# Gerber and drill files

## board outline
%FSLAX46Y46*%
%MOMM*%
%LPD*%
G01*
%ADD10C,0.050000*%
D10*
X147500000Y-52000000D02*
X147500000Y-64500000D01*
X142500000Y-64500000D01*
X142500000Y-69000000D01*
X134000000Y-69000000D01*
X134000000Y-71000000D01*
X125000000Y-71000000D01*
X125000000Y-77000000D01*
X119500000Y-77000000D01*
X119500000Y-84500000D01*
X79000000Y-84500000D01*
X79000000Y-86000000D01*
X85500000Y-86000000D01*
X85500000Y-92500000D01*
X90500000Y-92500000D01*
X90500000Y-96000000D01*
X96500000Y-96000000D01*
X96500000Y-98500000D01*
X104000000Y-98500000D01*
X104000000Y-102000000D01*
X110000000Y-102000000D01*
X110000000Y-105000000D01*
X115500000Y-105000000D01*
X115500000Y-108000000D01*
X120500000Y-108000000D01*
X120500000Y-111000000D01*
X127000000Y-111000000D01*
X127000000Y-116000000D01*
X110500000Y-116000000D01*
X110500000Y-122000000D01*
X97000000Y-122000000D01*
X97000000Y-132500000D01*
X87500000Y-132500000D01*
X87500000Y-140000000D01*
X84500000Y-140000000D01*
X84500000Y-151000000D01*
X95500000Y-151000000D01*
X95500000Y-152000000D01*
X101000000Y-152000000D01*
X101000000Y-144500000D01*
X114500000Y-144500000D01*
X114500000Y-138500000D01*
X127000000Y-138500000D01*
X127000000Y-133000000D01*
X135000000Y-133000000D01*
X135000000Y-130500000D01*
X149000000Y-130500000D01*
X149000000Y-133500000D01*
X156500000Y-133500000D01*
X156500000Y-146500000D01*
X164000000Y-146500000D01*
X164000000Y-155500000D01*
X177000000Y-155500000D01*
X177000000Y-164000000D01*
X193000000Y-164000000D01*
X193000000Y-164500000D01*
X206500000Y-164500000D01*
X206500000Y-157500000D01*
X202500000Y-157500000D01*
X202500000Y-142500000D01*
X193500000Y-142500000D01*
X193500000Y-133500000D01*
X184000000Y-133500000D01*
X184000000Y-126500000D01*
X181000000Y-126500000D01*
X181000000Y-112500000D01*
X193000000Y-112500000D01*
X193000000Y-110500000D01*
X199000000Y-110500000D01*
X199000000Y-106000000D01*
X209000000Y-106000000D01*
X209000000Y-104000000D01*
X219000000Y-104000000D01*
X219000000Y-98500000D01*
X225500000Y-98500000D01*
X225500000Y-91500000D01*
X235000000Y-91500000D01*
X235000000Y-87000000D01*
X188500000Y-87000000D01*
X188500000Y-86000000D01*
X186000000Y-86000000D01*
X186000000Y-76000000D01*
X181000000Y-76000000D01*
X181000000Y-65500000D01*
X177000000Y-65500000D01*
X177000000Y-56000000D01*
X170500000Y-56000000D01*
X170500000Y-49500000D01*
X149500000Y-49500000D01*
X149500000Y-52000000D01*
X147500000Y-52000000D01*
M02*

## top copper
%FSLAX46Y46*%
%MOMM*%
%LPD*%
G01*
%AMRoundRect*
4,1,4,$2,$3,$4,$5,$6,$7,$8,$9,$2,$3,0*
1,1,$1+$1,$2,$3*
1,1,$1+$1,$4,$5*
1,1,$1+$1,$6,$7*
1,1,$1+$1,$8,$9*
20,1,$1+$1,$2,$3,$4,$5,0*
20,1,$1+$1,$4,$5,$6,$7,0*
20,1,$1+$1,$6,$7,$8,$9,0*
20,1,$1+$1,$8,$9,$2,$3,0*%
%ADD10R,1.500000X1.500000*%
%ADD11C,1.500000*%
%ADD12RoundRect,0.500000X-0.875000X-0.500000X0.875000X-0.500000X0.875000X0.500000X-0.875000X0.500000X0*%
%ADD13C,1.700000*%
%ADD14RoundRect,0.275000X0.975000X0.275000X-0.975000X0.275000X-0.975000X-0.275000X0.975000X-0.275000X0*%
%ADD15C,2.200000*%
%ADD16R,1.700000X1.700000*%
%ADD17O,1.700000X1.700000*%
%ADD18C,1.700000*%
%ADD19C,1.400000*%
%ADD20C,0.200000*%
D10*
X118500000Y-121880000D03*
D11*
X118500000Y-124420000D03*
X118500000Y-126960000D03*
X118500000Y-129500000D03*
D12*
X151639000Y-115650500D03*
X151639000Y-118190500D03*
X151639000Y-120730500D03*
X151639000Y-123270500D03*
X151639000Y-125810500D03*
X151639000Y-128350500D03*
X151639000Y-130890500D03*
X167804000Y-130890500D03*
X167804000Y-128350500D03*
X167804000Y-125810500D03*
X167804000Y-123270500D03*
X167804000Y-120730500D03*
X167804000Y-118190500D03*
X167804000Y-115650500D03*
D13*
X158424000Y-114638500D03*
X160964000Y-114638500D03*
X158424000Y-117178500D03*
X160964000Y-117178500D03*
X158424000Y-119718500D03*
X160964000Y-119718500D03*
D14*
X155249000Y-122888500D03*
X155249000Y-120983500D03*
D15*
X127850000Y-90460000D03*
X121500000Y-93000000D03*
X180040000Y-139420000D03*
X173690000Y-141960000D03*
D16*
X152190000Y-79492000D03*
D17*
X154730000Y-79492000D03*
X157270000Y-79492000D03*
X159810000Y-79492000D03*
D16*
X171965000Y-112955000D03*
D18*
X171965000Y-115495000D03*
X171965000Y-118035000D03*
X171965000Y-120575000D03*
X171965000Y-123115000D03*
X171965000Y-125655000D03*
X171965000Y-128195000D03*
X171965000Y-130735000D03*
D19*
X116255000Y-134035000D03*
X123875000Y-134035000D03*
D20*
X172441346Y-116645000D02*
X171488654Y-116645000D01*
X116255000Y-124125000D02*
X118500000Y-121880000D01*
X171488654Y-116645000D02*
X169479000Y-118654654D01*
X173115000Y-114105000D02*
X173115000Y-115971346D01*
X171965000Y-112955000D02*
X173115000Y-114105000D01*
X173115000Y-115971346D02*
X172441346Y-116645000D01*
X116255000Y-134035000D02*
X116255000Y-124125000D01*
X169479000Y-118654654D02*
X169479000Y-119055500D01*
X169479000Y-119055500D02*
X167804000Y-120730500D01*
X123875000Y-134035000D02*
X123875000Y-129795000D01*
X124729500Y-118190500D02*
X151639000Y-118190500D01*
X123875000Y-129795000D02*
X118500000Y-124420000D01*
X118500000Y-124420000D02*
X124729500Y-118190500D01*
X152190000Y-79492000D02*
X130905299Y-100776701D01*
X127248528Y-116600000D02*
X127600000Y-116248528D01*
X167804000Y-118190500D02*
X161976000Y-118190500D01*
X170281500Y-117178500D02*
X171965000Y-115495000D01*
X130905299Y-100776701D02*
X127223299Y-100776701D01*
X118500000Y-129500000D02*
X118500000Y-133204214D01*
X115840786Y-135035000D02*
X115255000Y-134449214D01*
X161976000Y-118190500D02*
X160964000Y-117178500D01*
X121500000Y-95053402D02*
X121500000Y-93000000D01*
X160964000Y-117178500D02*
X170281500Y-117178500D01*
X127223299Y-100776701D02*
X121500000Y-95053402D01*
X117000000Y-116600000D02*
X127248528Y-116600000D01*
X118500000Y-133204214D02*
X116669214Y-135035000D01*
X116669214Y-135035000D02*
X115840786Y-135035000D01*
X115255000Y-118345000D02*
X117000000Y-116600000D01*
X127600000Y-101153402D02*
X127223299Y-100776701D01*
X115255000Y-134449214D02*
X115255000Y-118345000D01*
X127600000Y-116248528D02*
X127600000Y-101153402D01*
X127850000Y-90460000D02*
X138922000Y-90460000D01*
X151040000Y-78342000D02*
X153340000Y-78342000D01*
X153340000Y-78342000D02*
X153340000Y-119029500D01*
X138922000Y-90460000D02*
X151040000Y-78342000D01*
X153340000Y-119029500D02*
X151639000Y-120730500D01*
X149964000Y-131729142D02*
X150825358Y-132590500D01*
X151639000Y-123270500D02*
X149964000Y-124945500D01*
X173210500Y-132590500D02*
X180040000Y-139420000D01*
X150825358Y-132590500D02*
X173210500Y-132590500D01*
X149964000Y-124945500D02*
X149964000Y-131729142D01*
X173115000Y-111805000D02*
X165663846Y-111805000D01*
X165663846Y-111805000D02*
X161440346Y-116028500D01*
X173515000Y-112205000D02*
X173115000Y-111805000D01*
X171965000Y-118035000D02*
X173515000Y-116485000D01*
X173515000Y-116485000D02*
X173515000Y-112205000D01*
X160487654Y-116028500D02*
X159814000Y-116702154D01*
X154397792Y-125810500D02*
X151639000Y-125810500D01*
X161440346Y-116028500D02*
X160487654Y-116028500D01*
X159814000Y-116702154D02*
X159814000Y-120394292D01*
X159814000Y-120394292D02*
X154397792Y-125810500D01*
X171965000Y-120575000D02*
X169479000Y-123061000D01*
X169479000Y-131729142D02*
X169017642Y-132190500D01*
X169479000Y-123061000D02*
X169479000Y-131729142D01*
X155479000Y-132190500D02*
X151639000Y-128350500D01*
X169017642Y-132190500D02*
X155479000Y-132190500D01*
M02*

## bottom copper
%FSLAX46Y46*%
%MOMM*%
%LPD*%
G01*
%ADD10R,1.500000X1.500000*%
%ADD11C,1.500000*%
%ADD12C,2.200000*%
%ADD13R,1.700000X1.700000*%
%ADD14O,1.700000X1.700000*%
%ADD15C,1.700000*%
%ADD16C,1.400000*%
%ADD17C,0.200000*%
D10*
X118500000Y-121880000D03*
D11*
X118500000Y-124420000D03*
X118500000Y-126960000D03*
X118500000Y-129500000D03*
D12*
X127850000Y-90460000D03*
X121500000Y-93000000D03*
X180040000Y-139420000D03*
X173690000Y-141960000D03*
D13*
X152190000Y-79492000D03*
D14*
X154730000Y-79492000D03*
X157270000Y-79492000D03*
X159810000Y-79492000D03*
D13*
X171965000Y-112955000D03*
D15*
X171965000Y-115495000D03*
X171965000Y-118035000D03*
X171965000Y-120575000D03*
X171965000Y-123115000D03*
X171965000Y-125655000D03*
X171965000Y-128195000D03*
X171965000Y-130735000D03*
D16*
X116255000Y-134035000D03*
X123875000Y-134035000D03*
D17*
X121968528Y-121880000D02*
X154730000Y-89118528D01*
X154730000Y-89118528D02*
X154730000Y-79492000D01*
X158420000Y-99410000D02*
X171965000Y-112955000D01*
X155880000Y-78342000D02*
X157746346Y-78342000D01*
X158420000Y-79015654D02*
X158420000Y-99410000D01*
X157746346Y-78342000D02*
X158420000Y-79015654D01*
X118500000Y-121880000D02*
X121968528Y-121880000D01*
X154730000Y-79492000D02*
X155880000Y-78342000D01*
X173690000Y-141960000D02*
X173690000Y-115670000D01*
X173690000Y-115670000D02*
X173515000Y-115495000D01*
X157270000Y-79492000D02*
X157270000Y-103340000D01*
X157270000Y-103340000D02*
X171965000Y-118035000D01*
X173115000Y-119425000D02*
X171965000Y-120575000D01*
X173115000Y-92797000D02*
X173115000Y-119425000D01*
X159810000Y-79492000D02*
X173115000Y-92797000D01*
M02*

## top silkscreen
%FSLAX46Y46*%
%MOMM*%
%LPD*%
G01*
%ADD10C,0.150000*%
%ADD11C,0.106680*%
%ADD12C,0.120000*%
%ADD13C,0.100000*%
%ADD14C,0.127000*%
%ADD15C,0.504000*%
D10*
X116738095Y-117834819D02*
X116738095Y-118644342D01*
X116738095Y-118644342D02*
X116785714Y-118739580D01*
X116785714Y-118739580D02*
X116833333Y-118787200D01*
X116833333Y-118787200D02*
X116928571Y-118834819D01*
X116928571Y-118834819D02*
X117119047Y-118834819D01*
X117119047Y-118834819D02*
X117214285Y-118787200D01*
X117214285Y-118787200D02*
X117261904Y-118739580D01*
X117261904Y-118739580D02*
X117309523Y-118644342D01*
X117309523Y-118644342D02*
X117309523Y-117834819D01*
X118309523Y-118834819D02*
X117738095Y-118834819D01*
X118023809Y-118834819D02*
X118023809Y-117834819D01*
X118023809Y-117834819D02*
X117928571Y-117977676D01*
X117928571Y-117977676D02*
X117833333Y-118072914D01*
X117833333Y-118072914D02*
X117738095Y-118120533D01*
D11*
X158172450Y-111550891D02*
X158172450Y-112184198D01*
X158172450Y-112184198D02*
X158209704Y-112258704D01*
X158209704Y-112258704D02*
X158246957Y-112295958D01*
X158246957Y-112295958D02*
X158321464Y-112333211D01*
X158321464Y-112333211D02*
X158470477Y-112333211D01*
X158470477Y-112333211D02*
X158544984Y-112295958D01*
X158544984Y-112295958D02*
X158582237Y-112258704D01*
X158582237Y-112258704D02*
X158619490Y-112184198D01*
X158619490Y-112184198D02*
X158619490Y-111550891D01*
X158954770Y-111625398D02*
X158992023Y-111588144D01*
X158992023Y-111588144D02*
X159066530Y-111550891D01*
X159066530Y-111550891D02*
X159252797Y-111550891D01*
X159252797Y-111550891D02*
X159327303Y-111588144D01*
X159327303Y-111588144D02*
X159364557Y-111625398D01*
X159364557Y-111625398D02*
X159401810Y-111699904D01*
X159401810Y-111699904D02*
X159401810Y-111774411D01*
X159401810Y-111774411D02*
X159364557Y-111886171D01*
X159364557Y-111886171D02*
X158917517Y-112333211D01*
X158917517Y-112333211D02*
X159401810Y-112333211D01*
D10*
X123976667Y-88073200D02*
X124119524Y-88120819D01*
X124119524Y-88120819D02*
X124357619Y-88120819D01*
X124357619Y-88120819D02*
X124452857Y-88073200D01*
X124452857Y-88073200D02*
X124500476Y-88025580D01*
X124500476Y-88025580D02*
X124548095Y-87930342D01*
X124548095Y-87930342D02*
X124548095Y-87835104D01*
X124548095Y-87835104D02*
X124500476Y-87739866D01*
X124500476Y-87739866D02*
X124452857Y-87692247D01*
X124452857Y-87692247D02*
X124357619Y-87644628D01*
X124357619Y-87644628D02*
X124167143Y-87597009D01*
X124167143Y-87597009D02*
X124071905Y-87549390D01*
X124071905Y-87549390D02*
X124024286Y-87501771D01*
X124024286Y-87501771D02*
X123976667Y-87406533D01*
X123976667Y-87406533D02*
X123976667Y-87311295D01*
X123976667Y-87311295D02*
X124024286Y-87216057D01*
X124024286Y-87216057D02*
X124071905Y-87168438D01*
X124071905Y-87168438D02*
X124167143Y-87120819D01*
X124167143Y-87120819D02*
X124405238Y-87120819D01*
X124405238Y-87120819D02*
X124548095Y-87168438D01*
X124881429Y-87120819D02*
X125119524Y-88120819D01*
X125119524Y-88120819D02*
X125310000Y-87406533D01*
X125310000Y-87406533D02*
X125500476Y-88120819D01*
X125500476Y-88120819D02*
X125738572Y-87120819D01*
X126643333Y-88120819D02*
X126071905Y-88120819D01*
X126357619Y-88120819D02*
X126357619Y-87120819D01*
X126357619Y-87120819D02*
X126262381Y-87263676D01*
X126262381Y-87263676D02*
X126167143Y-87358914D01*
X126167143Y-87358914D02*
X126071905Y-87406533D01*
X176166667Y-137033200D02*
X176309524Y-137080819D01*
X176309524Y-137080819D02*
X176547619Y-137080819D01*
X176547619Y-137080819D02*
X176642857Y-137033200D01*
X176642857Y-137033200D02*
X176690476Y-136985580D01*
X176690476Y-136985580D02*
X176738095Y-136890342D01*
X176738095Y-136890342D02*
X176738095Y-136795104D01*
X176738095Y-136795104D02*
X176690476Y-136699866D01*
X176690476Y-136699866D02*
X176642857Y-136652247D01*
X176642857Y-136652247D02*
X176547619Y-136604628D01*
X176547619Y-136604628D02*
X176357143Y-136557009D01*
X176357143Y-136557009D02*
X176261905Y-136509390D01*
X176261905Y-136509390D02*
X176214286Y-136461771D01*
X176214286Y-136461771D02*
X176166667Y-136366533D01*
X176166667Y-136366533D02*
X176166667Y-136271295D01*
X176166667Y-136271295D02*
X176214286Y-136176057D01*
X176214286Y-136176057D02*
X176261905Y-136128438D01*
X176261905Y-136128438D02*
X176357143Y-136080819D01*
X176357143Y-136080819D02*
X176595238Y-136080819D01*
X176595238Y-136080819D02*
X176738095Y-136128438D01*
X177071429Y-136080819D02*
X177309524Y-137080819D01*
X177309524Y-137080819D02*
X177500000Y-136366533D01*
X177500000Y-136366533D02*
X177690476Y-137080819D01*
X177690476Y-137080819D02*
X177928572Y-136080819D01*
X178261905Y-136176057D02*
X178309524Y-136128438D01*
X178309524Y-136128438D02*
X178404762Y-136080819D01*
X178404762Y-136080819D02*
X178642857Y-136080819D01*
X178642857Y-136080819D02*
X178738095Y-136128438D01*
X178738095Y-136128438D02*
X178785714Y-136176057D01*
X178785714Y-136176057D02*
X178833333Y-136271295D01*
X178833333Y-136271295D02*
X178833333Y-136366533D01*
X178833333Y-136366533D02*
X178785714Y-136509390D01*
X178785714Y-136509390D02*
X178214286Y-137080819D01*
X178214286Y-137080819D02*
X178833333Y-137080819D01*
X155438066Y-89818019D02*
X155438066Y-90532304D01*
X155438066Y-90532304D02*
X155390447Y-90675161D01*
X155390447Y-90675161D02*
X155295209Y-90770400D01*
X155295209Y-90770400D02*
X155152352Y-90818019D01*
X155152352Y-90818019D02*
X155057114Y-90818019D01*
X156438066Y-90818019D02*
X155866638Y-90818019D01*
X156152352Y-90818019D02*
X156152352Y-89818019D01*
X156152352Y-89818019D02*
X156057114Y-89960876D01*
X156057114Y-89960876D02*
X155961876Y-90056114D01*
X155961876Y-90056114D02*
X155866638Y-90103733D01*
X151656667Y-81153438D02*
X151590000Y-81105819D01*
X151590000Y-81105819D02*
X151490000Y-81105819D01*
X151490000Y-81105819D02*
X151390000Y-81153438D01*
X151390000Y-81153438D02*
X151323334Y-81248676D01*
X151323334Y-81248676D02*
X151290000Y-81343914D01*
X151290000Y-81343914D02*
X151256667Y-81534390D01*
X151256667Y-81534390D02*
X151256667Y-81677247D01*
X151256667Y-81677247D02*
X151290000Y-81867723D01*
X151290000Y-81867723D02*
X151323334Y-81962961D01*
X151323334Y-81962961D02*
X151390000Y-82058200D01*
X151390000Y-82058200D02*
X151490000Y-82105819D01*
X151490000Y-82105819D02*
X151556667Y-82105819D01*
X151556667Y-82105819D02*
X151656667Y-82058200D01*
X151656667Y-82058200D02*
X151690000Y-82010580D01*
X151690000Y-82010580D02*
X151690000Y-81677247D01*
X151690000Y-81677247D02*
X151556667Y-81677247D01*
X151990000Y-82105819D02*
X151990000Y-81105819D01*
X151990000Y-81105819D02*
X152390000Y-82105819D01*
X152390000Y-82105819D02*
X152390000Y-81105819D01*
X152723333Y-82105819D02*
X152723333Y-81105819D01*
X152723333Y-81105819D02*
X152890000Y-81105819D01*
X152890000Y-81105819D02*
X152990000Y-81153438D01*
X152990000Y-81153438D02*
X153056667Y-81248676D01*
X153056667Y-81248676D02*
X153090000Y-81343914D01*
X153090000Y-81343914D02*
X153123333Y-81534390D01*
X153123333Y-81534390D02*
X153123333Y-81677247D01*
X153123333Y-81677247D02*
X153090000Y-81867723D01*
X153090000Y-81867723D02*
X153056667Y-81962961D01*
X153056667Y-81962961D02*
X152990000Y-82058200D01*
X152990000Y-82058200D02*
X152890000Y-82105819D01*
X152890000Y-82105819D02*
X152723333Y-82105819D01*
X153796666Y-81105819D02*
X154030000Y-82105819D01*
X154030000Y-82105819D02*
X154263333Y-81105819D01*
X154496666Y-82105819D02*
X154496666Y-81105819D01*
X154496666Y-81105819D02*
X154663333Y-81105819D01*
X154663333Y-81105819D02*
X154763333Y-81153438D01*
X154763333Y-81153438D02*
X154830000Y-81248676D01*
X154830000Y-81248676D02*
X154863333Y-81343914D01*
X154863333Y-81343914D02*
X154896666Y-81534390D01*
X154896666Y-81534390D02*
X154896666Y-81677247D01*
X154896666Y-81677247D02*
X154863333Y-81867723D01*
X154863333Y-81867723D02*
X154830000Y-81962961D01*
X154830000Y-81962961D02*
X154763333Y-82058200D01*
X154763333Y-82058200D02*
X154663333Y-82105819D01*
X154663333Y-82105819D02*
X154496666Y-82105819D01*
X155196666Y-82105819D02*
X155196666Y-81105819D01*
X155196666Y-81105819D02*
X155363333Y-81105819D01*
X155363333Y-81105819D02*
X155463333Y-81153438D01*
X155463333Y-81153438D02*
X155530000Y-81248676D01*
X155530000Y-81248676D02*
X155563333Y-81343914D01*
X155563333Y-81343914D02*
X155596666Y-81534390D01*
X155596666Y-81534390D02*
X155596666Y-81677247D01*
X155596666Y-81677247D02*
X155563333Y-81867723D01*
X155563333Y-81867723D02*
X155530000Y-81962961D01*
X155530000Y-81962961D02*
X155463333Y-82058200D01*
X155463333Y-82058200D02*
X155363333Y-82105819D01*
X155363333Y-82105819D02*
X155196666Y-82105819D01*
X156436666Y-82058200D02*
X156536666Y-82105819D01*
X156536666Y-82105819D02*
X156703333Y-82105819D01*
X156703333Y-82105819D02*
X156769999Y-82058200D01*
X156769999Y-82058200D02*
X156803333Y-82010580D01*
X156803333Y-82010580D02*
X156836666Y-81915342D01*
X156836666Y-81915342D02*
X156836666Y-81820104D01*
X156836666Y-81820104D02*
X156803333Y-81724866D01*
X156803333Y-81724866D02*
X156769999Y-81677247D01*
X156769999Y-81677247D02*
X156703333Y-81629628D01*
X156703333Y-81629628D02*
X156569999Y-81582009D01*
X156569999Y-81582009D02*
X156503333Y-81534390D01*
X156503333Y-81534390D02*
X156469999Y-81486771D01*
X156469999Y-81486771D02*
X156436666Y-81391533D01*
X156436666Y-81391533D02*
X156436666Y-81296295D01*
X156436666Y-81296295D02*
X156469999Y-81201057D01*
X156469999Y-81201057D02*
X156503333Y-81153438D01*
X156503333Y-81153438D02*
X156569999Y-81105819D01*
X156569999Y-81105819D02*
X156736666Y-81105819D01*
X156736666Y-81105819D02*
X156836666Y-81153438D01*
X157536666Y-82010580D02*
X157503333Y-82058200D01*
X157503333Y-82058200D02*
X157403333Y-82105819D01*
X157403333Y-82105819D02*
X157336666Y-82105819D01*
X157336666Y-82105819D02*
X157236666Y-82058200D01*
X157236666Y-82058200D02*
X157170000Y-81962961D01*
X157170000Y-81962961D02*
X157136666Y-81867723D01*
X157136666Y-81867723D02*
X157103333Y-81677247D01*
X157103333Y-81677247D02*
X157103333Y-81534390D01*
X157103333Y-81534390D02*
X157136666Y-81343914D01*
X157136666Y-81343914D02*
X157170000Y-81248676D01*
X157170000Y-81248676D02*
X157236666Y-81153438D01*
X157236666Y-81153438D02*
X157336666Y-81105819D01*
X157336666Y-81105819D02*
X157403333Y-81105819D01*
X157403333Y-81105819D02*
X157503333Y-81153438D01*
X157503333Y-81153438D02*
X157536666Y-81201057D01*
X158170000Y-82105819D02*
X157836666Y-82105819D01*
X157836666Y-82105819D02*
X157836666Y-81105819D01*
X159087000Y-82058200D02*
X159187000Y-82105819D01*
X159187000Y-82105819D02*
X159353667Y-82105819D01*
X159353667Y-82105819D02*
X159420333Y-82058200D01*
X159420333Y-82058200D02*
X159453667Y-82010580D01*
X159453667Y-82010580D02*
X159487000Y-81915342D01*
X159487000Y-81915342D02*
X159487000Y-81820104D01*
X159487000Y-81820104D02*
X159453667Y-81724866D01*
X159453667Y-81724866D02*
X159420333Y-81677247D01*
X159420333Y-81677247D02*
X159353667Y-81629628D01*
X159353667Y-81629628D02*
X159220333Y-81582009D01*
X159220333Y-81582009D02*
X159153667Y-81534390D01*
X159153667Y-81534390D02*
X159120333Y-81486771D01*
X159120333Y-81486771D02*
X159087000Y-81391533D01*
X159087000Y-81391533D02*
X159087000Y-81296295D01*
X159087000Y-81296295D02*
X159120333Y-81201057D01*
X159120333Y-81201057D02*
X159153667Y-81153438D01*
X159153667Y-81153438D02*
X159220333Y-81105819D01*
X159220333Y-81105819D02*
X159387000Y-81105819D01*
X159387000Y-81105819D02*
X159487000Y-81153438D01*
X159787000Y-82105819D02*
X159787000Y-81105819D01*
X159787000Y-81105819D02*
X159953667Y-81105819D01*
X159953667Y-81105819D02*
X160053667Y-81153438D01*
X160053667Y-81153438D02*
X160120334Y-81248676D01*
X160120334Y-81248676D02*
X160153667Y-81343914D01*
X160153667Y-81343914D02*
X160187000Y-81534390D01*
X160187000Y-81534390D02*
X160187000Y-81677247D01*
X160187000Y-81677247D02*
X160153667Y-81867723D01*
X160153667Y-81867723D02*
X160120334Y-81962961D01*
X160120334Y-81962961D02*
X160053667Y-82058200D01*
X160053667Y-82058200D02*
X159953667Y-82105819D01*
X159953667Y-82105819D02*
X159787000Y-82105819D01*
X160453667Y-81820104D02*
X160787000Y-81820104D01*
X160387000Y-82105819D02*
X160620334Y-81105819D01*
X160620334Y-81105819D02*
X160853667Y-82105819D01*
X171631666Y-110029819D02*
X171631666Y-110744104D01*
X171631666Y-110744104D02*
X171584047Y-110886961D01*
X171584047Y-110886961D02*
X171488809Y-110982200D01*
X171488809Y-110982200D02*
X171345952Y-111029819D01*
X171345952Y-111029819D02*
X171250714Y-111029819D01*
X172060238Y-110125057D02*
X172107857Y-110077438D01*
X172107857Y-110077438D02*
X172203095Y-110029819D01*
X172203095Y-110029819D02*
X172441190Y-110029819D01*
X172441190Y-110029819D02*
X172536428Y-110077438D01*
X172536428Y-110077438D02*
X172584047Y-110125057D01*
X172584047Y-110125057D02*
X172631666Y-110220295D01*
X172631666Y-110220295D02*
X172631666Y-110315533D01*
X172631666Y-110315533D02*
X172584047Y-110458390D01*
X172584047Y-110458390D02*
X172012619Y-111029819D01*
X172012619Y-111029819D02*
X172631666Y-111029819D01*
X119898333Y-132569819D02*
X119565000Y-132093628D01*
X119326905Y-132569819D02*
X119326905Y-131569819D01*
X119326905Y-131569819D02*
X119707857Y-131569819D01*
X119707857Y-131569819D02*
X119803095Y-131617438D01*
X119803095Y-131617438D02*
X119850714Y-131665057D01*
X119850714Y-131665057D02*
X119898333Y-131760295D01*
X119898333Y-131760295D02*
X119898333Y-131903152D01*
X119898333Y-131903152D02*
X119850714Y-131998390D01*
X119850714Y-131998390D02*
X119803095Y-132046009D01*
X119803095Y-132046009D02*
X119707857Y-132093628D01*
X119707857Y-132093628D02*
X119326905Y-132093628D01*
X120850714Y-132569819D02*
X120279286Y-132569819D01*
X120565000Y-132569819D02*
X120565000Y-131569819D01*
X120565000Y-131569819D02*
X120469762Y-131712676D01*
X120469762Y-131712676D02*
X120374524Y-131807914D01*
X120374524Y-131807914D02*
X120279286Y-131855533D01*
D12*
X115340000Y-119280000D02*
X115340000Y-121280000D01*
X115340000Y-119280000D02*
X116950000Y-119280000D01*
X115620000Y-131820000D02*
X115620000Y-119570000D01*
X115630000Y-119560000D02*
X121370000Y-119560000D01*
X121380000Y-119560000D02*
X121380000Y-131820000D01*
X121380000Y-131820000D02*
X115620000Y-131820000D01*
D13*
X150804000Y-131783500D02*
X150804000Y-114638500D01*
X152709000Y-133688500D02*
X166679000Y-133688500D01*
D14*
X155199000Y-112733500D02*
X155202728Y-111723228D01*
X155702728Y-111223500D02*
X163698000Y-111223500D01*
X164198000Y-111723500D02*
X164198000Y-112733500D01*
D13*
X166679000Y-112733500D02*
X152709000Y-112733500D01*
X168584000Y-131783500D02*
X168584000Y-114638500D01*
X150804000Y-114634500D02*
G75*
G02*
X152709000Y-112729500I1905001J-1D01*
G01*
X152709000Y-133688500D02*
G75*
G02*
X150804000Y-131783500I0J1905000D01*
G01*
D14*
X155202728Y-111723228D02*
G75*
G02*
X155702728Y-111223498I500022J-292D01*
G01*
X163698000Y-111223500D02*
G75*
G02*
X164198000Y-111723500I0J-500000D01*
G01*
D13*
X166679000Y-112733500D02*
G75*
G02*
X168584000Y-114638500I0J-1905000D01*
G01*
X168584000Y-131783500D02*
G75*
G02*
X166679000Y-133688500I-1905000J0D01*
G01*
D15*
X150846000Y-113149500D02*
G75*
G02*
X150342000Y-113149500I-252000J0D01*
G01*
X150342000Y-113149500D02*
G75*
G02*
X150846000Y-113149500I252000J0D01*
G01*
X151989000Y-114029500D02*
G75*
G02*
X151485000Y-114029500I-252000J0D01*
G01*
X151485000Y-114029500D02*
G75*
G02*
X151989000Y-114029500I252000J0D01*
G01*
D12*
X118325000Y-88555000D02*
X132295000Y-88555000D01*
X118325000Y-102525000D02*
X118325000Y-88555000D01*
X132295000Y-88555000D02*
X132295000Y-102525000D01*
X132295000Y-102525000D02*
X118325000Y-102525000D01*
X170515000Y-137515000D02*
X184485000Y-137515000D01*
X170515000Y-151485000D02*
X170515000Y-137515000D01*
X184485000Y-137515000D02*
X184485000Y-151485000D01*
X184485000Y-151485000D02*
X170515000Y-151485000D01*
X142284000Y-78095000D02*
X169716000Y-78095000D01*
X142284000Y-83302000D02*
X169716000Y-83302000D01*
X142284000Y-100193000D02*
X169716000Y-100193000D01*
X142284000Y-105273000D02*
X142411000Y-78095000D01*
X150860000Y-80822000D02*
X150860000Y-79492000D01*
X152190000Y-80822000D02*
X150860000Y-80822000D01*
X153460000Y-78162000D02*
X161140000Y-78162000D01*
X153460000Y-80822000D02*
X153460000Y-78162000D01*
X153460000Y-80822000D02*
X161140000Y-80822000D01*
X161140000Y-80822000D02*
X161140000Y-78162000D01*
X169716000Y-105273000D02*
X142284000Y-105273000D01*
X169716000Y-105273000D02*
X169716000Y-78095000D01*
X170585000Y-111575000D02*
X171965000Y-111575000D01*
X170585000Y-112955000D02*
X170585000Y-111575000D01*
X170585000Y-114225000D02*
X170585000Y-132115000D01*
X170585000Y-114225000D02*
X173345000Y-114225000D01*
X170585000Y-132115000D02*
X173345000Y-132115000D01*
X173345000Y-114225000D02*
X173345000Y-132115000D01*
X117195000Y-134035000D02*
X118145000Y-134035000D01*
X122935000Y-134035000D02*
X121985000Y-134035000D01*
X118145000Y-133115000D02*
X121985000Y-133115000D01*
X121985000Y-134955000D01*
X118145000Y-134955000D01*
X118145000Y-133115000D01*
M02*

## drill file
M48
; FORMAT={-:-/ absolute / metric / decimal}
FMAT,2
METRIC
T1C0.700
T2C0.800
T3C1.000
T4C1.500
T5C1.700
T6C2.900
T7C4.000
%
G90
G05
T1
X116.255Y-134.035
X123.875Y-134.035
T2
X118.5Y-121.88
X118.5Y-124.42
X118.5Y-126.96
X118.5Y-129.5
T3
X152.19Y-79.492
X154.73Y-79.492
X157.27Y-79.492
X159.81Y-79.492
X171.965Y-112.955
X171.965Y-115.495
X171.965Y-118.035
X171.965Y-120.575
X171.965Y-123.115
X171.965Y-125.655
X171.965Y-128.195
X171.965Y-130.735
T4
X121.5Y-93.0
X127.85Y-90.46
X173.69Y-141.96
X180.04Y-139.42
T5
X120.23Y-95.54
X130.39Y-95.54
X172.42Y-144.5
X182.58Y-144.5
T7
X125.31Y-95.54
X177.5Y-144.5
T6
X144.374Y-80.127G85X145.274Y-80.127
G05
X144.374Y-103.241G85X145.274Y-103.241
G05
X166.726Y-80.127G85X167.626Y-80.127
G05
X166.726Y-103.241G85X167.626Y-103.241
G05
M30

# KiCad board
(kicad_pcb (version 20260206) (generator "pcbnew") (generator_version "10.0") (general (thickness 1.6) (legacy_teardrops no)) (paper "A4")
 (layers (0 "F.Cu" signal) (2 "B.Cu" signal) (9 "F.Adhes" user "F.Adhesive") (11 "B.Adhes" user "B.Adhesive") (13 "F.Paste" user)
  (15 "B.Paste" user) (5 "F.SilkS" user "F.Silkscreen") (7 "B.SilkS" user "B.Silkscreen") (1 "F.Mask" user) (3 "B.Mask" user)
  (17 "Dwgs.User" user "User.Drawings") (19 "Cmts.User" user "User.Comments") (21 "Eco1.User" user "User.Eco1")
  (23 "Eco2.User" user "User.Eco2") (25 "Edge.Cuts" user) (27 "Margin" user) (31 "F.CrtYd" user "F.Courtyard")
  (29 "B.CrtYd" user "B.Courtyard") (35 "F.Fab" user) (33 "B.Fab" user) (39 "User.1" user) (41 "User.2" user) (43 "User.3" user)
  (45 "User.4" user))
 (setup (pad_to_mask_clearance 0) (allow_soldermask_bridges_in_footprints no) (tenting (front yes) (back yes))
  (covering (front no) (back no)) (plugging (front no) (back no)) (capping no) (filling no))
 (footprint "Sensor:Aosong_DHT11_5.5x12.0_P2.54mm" (layer "F.Cu") (at 118.5 121.88)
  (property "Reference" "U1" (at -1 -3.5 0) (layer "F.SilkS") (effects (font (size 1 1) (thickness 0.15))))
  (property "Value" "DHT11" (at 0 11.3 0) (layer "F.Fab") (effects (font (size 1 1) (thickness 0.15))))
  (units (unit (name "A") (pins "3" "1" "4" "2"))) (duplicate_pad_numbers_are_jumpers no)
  (fp_line (start -3.16 -2.6) (end -3.16 -0.6) (stroke (width 0.12) (type solid)) (layer "F.SilkS"))
  (fp_line (start -3.16 -2.6) (end -1.55 -2.6) (stroke (width 0.12) (type solid)) (layer "F.SilkS"))
  (fp_line (start -2.88 9.94) (end -2.88 -2.31) (stroke (width 0.12) (type solid)) (layer "F.SilkS"))
  (fp_line (start -2.87 -2.32) (end 2.87 -2.32) (stroke (width 0.12) (type solid)) (layer "F.SilkS"))
  (fp_line (start 2.88 -2.32) (end 2.88 9.94) (stroke (width 0.12) (type solid)) (layer "F.SilkS"))
  (fp_line (start 2.88 9.94) (end -2.88 9.94) (stroke (width 0.12) (type solid)) (layer "F.SilkS"))
  (pad "1" thru_hole rect (at 0 0) (size 1.5 1.5) (drill 0.8) (layers "*.Cu" "*.Mask") (remove_unused_layers no) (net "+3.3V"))
  (pad "2" thru_hole circle (at 0 2.54) (size 1.5 1.5) (drill 0.8) (layers "*.Cu" "*.Mask") (remove_unused_layers no) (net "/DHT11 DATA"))
  (pad "3" thru_hole circle (at 0 5.08) (size 1.5 1.5) (drill 0.8) (layers "*.Cu" "*.Mask") (remove_unused_layers no)
   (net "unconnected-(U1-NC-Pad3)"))
  (pad "4" thru_hole circle (at 0 7.62) (size 1.5 1.5) (drill 0.8) (layers "*.Cu" "*.Mask") (remove_unused_layers no) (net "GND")))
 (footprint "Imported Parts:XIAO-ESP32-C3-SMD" (layer "F.Cu") (at 150.804 133.7705)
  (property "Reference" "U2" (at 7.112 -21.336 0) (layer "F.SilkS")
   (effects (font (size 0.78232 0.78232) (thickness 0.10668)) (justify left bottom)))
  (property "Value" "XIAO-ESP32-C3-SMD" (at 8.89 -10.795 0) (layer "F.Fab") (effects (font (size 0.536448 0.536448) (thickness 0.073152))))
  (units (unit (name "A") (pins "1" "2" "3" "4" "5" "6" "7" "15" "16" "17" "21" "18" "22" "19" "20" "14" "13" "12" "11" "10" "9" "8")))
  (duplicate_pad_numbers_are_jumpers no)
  (fp_line (start 0 -1.987) (end 0 -19.132) (stroke (width 0.1) (type solid)) (layer "F.SilkS"))
  (fp_line (start 1.905 -0.082) (end 15.875 -0.082) (stroke (width 0.1) (type solid)) (layer "F.SilkS"))
  (fp_line (start 4.395 -21.037) (end 4.398728 -22.047272) (stroke (width 0.127) (type solid)) (layer "F.SilkS"))
  (fp_line (start 4.898728 -22.547) (end 12.894 -22.547) (stroke (width 0.127) (type solid)) (layer "F.SilkS"))
  (fp_line (start 13.394 -22.047) (end 13.394 -21.037) (stroke (width 0.127) (type solid)) (layer "F.SilkS"))
  (fp_line (start 15.875 -21.037) (end 1.905 -21.037) (stroke (width 0.1) (type solid)) (layer "F.SilkS"))
  (fp_line (start 17.78 -1.987) (end 17.78 -19.132) (stroke (width 0.1) (type solid)) (layer "F.SilkS"))
  (fp_arc (start 0 -19.136) (mid 0.557962 -20.483038) (end 1.905 -21.041) (stroke (width 0.1) (type solid)) (layer "F.SilkS"))
  (fp_arc (start 1.905 -0.082) (mid 0.557962 -0.639962) (end 0 -1.987) (stroke (width 0.1) (type solid)) (layer "F.SilkS"))
  (fp_arc (start 4.398728 -22.047272) (mid 4.545272 -22.40064) (end 4.898728 -22.547) (stroke (width 0.127) (type default))
   (layer "F.SilkS"))
  (fp_arc (start 12.894 -22.547) (mid 13.247553 -22.400553) (end 13.394 -22.047) (stroke (width 0.127) (type default)) (layer "F.SilkS"))
  (fp_arc (start 15.875 -21.037) (mid 17.222038 -20.479038) (end 17.78 -19.132) (stroke (width 0.1) (type solid)) (layer "F.SilkS"))
  (fp_arc (start 17.78 -1.987) (mid 17.222038 -0.639962) (end 15.875 -0.082) (stroke (width 0.1) (type solid)) (layer "F.SilkS"))
  (fp_circle (center -0.21 -20.621) (end -0.21 -20.875) (stroke (width 0.5) (type solid)) (fill yes) (layer "F.SilkS"))
  (fp_circle (center 0.933 -19.741) (end 0.933 -19.995) (stroke (width 0.5) (type solid)) (fill yes) (layer "F.SilkS"))
  (pad "1" smd roundrect (at 0.835 -18.12) (size 2.75 2) (layers "F.Cu" "F.Mask" "F.Paste") (roundrect_rratio 0.25)
   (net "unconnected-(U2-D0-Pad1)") (solder_mask_margin 0.0508) (thermal_bridge_angle 45))
  (pad "2" smd roundrect (at 0.835 -15.58) (size 2.75 2) (layers "F.Cu" "F.Mask" "F.Paste") (roundrect_rratio 0.25) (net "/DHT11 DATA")
   (solder_mask_margin 0.0508) (thermal_bridge_angle 45))
  (pad "3" smd roundrect (at 0.835 -13.04) (size 2.75 2) (layers "F.Cu" "F.Mask" "F.Paste") (roundrect_rratio 0.25) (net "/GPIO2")
   (solder_mask_margin 0.0508) (thermal_bridge_angle 45))
  (pad "4" smd roundrect (at 0.835 -10.5) (size 2.75 2) (layers "F.Cu" "F.Mask" "F.Paste") (roundrect_rratio 0.25) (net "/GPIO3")
   (solder_mask_margin 0.0508) (thermal_bridge_angle 45))
  (pad "5" smd roundrect (at 0.835 -7.96) (size 2.75 2) (layers "F.Cu" "F.Mask" "F.Paste") (roundrect_rratio 0.25) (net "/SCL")
   (solder_mask_margin 0.0508) (thermal_bridge_angle 45))
  (pad "6" smd roundrect (at 0.835 -5.42) (size 2.75 2) (layers "F.Cu" "F.Mask" "F.Paste") (roundrect_rratio 0.25) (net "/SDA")
   (solder_mask_margin 0.0508) (thermal_bridge_angle 45))
  (pad "7" smd roundrect (at 0.835 -2.88) (size 2.75 2) (layers "F.Cu" "F.Mask" "F.Paste") (roundrect_rratio 0.25)
   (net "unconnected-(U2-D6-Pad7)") (solder_mask_margin 0.0508) (thermal_bridge_angle 45))
  (pad "8" smd roundrect (at 17 -2.88) (size 2.75 2) (layers "F.Cu" "F.Mask" "F.Paste") (roundrect_rratio 0.25)
   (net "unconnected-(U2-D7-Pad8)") (solder_mask_margin 0.0508) (thermal_bridge_angle 45))
  (pad "9" smd roundrect (at 17 -5.42) (size 2.75 2) (layers "F.Cu" "F.Mask" "F.Paste") (roundrect_rratio 0.25)
   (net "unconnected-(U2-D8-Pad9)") (solder_mask_margin 0.0508) (thermal_bridge_angle 45))
  (pad "10" smd roundrect (at 17 -7.96) (size 2.75 2) (layers "F.Cu" "F.Mask" "F.Paste") (roundrect_rratio 0.25)
   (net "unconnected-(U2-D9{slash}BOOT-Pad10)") (solder_mask_margin 0.0508) (thermal_bridge_angle 45))
  (pad "11" smd roundrect (at 17 -10.5) (size 2.75 2) (layers "F.Cu" "F.Mask" "F.Paste") (roundrect_rratio 0.25)
   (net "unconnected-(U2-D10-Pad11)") (solder_mask_margin 0.0508) (thermal_bridge_angle 45))
  (pad "12" smd roundrect (at 17 -13.04) (size 2.75 2) (layers "F.Cu" "F.Mask" "F.Paste") (roundrect_rratio 0.25) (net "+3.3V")
   (solder_mask_margin 0.0508) (thermal_bridge_angle 45))
  (pad "13" smd roundrect (at 17 -15.58) (size 2.75 2) (layers "F.Cu" "F.Mask" "F.Paste") (roundrect_rratio 0.25) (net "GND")
   (solder_mask_margin 0.0508) (thermal_bridge_angle 45))
  (pad "14" smd roundrect (at 17 -18.12) (size 2.75 2) (layers "F.Cu" "F.Mask" "F.Paste") (roundrect_rratio 0.25) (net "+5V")
   (solder_mask_margin 0.0508) (thermal_bridge_angle 45))
  (pad "15" smd circle (at 7.62 -19.132) (size 1.7 1.7) (layers "F.Cu" "F.Mask" "F.Paste") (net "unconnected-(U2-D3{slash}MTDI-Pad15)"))
  (pad "16" smd circle (at 10.16 -19.132) (size 1.7 1.7) (layers "F.Cu" "F.Mask" "F.Paste") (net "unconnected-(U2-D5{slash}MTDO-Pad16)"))
  (pad "17" smd circle (at 7.62 -16.592) (size 1.7 1.7) (layers "F.Cu" "F.Mask" "F.Paste") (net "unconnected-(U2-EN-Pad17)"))
  (pad "18" smd circle (at 10.16 -16.592) (size 1.7 1.7) (layers "F.Cu" "F.Mask" "F.Paste") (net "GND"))
  (pad "19" smd circle (at 7.62 -14.052) (size 1.7 1.7) (layers "F.Cu" "F.Mask" "F.Paste") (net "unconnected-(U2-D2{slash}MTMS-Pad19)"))
  (pad "20" smd circle (at 10.16 -14.052) (size 1.7 1.7) (layers "F.Cu" "F.Mask" "F.Paste") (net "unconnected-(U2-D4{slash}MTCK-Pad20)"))
  (pad "21" smd roundrect (at 4.445 -10.882 180) (size 2.5 1.1) (layers "F.Cu" "F.Mask" "F.Paste") (roundrect_rratio 0.25)
   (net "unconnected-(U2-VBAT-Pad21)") (thermal_bridge_angle 45))
  (pad "22" smd roundrect (at 4.445 -12.787 180) (size 2.5 1.1) (layers "F.Cu" "F.Mask" "F.Paste") (roundrect_rratio 0.25)
   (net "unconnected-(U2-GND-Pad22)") (thermal_bridge_angle 45)))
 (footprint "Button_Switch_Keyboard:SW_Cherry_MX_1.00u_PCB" (layer "F.Cu") (at 127.85 90.46)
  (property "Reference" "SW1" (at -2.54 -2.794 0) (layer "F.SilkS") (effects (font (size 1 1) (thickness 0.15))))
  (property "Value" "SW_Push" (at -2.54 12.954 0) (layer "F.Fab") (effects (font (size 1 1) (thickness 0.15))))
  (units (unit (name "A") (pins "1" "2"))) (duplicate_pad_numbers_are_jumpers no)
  (fp_line (start -9.525 -1.905) (end 4.445 -1.905) (stroke (width 0.12) (type solid)) (layer "F.SilkS"))
  (fp_line (start -9.525 12.065) (end -9.525 -1.905) (stroke (width 0.12) (type solid)) (layer "F.SilkS"))
  (fp_line (start 4.445 -1.905) (end 4.445 12.065) (stroke (width 0.12) (type solid)) (layer "F.SilkS"))
  (fp_line (start 4.445 12.065) (end -9.525 12.065) (stroke (width 0.12) (type solid)) (layer "F.SilkS"))
  (pad "" np_thru_hole circle (at -7.62 5.08) (size 1.7 1.7) (drill 1.7) (layers "*.Cu" "*.Mask"))
  (pad "" np_thru_hole circle (at -2.54 5.08) (size 4 4) (drill 4) (layers "*.Cu" "*.Mask"))
  (pad "" np_thru_hole circle (at 2.54 5.08) (size 1.7 1.7) (drill 1.7) (layers "*.Cu" "*.Mask"))
  (pad "1" thru_hole circle (at 0 0) (size 2.2 2.2) (drill 1.5) (layers "*.Cu" "*.Mask") (remove_unused_layers no) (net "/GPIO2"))
  (pad "2" thru_hole circle (at -6.35 2.54) (size 2.2 2.2) (drill 1.5) (layers "*.Cu" "*.Mask") (remove_unused_layers no) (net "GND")))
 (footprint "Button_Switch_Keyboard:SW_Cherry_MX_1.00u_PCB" (layer "F.Cu") (at 180.04 139.42)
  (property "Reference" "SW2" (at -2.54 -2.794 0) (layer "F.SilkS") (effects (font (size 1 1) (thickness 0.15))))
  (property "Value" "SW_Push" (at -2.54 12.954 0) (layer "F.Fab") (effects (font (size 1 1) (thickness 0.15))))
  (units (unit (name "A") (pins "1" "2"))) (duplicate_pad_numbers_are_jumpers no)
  (fp_line (start -9.525 -1.905) (end 4.445 -1.905) (stroke (width 0.12) (type solid)) (layer "F.SilkS"))
  (fp_line (start -9.525 12.065) (end -9.525 -1.905) (stroke (width 0.12) (type solid)) (layer "F.SilkS"))
  (fp_line (start 4.445 -1.905) (end 4.445 12.065) (stroke (width 0.12) (type solid)) (layer "F.SilkS"))
  (fp_line (start 4.445 12.065) (end -9.525 12.065) (stroke (width 0.12) (type solid)) (layer "F.SilkS"))
  (pad "" np_thru_hole circle (at -7.62 5.08) (size 1.7 1.7) (drill 1.7) (layers "*.Cu" "*.Mask"))
  (pad "" np_thru_hole circle (at -2.54 5.08) (size 4 4) (drill 4) (layers "*.Cu" "*.Mask"))
  (pad "" np_thru_hole circle (at 2.54 5.08) (size 1.7 1.7) (drill 1.7) (layers "*.Cu" "*.Mask"))
  (pad "1" thru_hole circle (at 0 0) (size 2.2 2.2) (drill 1.5) (layers "*.Cu" "*.Mask") (remove_unused_layers no) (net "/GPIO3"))
  (pad "2" thru_hole circle (at -6.35 2.54) (size 2.2 2.2) (drill 1.5) (layers "*.Cu" "*.Mask") (remove_unused_layers no) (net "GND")))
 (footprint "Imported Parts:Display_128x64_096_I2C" (layer "F.Cu") (at 156 79.492)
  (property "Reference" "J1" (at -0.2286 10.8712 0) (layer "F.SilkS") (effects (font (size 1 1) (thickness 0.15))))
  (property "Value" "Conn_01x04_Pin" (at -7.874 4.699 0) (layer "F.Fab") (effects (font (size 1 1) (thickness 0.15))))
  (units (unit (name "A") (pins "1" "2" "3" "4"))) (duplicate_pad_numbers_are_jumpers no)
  (fp_line (start -13.716 -1.397) (end 13.716 -1.397) (stroke (width 0.12) (type solid)) (layer "F.SilkS"))
  (fp_line (start -13.716 3.81) (end 13.716 3.81) (stroke (width 0.12) (type solid)) (layer "F.SilkS"))
  (fp_line (start -13.716 20.701) (end 13.716 20.701) (stroke (width 0.12) (type solid)) (layer "F.SilkS"))
  (fp_line (start -13.716 25.781) (end -13.589 -1.397) (stroke (width 0.12) (type solid)) (layer "F.SilkS"))
  (fp_line (start -5.14 1.33) (end -5.14 0) (stroke (width 0.12) (type solid)) (layer "F.SilkS"))
  (fp_line (start -3.81 1.33) (end -5.14 1.33) (stroke (width 0.12) (type solid)) (layer "F.SilkS"))
  (fp_line (start -2.54 -1.33) (end 5.14 -1.33) (stroke (width 0.12) (type solid)) (layer "F.SilkS"))
  (fp_line (start -2.54 1.33) (end -2.54 -1.33) (stroke (width 0.12) (type solid)) (layer "F.SilkS"))
  (fp_line (start -2.54 1.33) (end 5.14 1.33) (stroke (width 0.12) (type solid)) (layer "F.SilkS"))
  (fp_line (start 5.14 1.33) (end 5.14 -1.33) (stroke (width 0.12) (type solid)) (layer "F.SilkS"))
  (fp_line (start 13.716 25.781) (end -13.716 25.781) (stroke (width 0.12) (type solid)) (layer "F.SilkS"))
  (fp_line (start 13.716 25.781) (end 13.716 -1.397) (stroke (width 0.12) (type solid)) (layer "F.SilkS"))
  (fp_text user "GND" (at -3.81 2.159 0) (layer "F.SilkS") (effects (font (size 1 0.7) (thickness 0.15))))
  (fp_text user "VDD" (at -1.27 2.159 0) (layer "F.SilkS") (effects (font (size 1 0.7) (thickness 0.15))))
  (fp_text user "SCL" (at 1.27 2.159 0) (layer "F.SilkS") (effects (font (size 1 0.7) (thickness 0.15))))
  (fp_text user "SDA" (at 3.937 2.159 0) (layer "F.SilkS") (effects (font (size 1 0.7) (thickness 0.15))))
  (pad "" np_thru_hole oval (at -11.176 0.635) (size 3.8 2.9) (drill oval 3.8 2.9) (layers "*.Cu" "*.Mask"))
  (pad "" np_thru_hole oval (at -11.176 23.749) (size 3.8 2.9) (drill oval 3.8 2.9) (layers "*.Cu" "*.Mask"))
  (pad "" np_thru_hole oval (at 11.176 0.635) (size 3.8 2.9) (drill oval 3.8 2.9) (layers "*.Cu" "*.Mask"))
  (pad "" np_thru_hole oval (at 11.176 23.749) (size 3.8 2.9) (drill oval 3.8 2.9) (layers "*.Cu" "*.Mask"))
  (pad "1" thru_hole rect (at -3.81 0 90) (size 1.7 1.7) (drill 1) (layers "*.Cu" "*.Mask") (remove_unused_layers no) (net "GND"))
  (pad "2" thru_hole oval (at -1.27 0 90) (size 1.7 1.7) (drill 1) (layers "*.Cu" "*.Mask") (remove_unused_layers no) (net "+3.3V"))
  (pad "3" thru_hole oval (at 1.27 0 90) (size 1.7 1.7) (drill 1) (layers "*.Cu" "*.Mask") (remove_unused_layers no) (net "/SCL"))
  (pad "4" thru_hole oval (at 3.81 0 90) (size 1.7 1.7) (drill 1) (layers "*.Cu" "*.Mask") (remove_unused_layers no) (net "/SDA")))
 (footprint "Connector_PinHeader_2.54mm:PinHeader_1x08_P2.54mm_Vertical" (layer "F.Cu") (at 171.965 112.955)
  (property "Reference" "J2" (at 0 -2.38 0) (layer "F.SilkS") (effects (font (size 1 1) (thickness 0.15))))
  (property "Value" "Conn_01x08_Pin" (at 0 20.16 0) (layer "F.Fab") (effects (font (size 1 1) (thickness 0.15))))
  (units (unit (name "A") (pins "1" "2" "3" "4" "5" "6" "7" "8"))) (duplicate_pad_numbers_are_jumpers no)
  (fp_line (start -1.38 -1.38) (end 0 -1.38) (stroke (width 0.12) (type solid)) (layer "F.SilkS"))
  (fp_line (start -1.38 0) (end -1.38 -1.38) (stroke (width 0.12) (type solid)) (layer "F.SilkS"))
  (fp_line (start -1.38 1.27) (end -1.38 19.16) (stroke (width 0.12) (type solid)) (layer "F.SilkS"))
  (fp_line (start -1.38 1.27) (end 1.38 1.27) (stroke (width 0.12) (type solid)) (layer "F.SilkS"))
  (fp_line (start -1.38 19.16) (end 1.38 19.16) (stroke (width 0.12) (type solid)) (layer "F.SilkS"))
  (fp_line (start 1.38 1.27) (end 1.38 19.16) (stroke (width 0.12) (type solid)) (layer "F.SilkS"))
  (pad "1" thru_hole rect (at 0 0) (size 1.7 1.7) (drill 1) (layers "*.Cu" "*.Mask") (remove_unused_layers no) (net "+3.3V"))
  (pad "2" thru_hole circle (at 0 2.54) (size 1.7 1.7) (drill 1) (layers "*.Cu" "*.Mask") (remove_unused_layers no) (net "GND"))
  (pad "3" thru_hole circle (at 0 5.08) (size 1.7 1.7) (drill 1) (layers "*.Cu" "*.Mask") (remove_unused_layers no) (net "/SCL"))
  (pad "4" thru_hole circle (at 0 7.62) (size 1.7 1.7) (drill 1) (layers "*.Cu" "*.Mask") (remove_unused_layers no) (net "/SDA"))
  (pad "5" thru_hole circle (at 0 10.16) (size 1.7 1.7) (drill 1) (layers "*.Cu" "*.Mask") (remove_unused_layers no)
   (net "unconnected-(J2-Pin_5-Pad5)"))
  (pad "6" thru_hole circle (at 0 12.7) (size 1.7 1.7) (drill 1) (layers "*.Cu" "*.Mask") (remove_unused_layers no)
   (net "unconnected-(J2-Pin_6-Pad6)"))
  (pad "7" thru_hole circle (at 0 15.24) (size 1.7 1.7) (drill 1) (layers "*.Cu" "*.Mask") (remove_unused_layers no)
   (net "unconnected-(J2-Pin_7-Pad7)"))
  (pad "8" thru_hole circle (at 0 17.78) (size 1.7 1.7) (drill 1) (layers "*.Cu" "*.Mask") (remove_unused_layers no)
   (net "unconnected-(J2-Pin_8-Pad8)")))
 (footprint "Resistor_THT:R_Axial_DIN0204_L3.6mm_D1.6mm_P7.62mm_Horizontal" (layer "F.Cu") (at 116.255 134.035)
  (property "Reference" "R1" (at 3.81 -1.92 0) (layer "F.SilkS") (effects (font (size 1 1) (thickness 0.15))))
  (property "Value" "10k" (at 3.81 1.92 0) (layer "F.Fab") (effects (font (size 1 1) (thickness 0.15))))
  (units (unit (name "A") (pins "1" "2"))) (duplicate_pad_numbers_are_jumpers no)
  (fp_line (start 0.94 0) (end 1.89 0) (stroke (width 0.12) (type solid)) (layer "F.SilkS"))
  (fp_line (start 6.68 0) (end 5.73 0) (stroke (width 0.12) (type solid)) (layer "F.SilkS"))
  (fp_rect (start 1.89 -0.92) (end 5.73 0.92) (stroke (width 0.12) (type solid)) (fill no) (layer "F.SilkS"))
  (pad "1" thru_hole circle (at 0 0) (size 1.4 1.4) (drill 0.7) (layers "*.Cu" "*.Mask") (remove_unused_layers no) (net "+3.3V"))
  (pad "2" thru_hole circle (at 7.62 0) (size 1.4 1.4) (drill 0.7) (layers "*.Cu" "*.Mask") (remove_unused_layers no) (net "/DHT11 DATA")))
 (gr_poly
  (pts (xy 147.5 52) (xy 147.5 64.5) (xy 142.5 64.5) (xy 142.5 69) (xy 134 69) (xy 134 71) (xy 125 71) (xy 125 77) (xy 119.5 77)
   (xy 119.5 84.5) (xy 79 84.5) (xy 79 86) (xy 85.5 86) (xy 85.5 92.5) (xy 90.5 92.5) (xy 90.5 96) (xy 96.5 96) (xy 96.5 98.5) (xy 104 98.5)
   (xy 104 102) (xy 110 102) (xy 110 105) (xy 115.5 105) (xy 115.5 108) (xy 120.5 108) (xy 120.5 111) (xy 127 111) (xy 127 116)
   (xy 110.5 116) (xy 110.5 122) (xy 97 122) (xy 97 132.5) (xy 87.5 132.5) (xy 87.5 140) (xy 84.5 140) (xy 84.5 151) (xy 95.5 151)
   (xy 95.5 152) (xy 101 152) (xy 101 144.5) (xy 114.5 144.5) (xy 114.5 138.5) (xy 127 138.5) (xy 127 133) (xy 135 133) (xy 135 130.5)
   (xy 149 130.5) (xy 149 133.5) (xy 156.5 133.5) (xy 156.5 146.5) (xy 164 146.5) (xy 164 155.5) (xy 177 155.5) (xy 177 164) (xy 193 164)
   (xy 193 164.5) (xy 206.5 164.5) (xy 206.5 157.5) (xy 202.5 157.5) (xy 202.5 142.5) (xy 193.5 142.5) (xy 193.5 133.5) (xy 184 133.5)
   (xy 184 126.5) (xy 181 126.5) (xy 181 112.5) (xy 193 112.5) (xy 193 110.5) (xy 199 110.5) (xy 199 106) (xy 209 106) (xy 209 104)
   (xy 219 104) (xy 219 98.5) (xy 225.5 98.5) (xy 225.5 91.5) (xy 235 91.5) (xy 235 87) (xy 188.5 87) (xy 188.5 86) (xy 186 86) (xy 186 76)
   (xy 181 76) (xy 181 65.5) (xy 177 65.5) (xy 177 56) (xy 170.5 56) (xy 170.5 49.5) (xy 149.5 49.5) (xy 149.5 52))
  (stroke (width 0.05) (type solid)) (fill no) (layer "Edge.Cuts"))
 (segment (start 172.441346 116.645) (end 171.488654 116.645) (width 0.2) (layer "F.Cu") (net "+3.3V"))
 (segment (start 116.255 124.125) (end 118.5 121.88) (width 0.2) (layer "F.Cu") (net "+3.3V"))
 (segment (start 171.488654 116.645) (end 169.479 118.654654) (width 0.2) (layer "F.Cu") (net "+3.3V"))
 (segment (start 173.115 114.105) (end 173.115 115.971346) (width 0.2) (layer "F.Cu") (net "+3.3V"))
 (segment (start 171.965 112.955) (end 173.115 114.105) (width 0.2) (layer "F.Cu") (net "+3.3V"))
 (segment (start 173.115 115.971346) (end 172.441346 116.645) (width 0.2) (layer "F.Cu") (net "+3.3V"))
 (segment (start 116.255 134.035) (end 116.255 124.125) (width 0.2) (layer "F.Cu") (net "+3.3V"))
 (segment (start 169.479 118.654654) (end 169.479 119.0555) (width 0.2) (layer "F.Cu") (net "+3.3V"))
 (segment (start 169.479 119.0555) (end 167.804 120.7305) (width 0.2) (layer "F.Cu") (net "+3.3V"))
 (segment (start 121.968528 121.88) (end 154.73 89.118528) (width 0.2) (layer "B.Cu") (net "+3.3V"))
 (segment (start 154.73 89.118528) (end 154.73 79.492) (width 0.2) (layer "B.Cu") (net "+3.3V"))
 (segment (start 158.42 99.41) (end 171.965 112.955) (width 0.2) (layer "B.Cu") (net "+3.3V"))
 (segment (start 155.88 78.342) (end 157.746346 78.342) (width 0.2) (layer "B.Cu") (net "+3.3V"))
 (segment (start 158.42 79.015654) (end 158.42 99.41) (width 0.2) (layer "B.Cu") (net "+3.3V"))
 (segment (start 157.746346 78.342) (end 158.42 79.015654) (width 0.2) (layer "B.Cu") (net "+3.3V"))
 (segment (start 118.5 121.88) (end 121.968528 121.88) (width 0.2) (layer "B.Cu") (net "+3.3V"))
 (segment (start 154.73 79.492) (end 155.88 78.342) (width 0.2) (layer "B.Cu") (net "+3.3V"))
 (segment (start 123.875 134.035) (end 123.875 129.795) (width 0.2) (layer "F.Cu") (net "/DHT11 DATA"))
 (segment (start 124.7295 118.1905) (end 151.639 118.1905) (width 0.2) (layer "F.Cu") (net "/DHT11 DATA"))
 (segment (start 123.875 129.795) (end 118.5 124.42) (width 0.2) (layer "F.Cu") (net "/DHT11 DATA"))
 (segment (start 118.5 124.42) (end 124.7295 118.1905) (width 0.2) (layer "F.Cu") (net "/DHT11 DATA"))
 (segment (start 152.19 79.492) (end 130.905299 100.776701) (width 0.2) (layer "F.Cu") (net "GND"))
 (segment (start 127.248528 116.6) (end 127.6 116.248528) (width 0.2) (layer "F.Cu") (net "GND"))
 (segment (start 167.804 118.1905) (end 161.976 118.1905) (width 0.2) (layer "F.Cu") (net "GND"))
 (segment (start 170.2815 117.1785) (end 171.965 115.495) (width 0.2) (layer "F.Cu") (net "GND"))
 (segment (start 130.905299 100.776701) (end 127.223299 100.776701) (width 0.2) (layer "F.Cu") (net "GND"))
 (segment (start 118.5 129.5) (end 118.5 133.204214) (width 0.2) (layer "F.Cu") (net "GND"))
 (segment (start 115.840786 135.035) (end 115.255 134.449214) (width 0.2) (layer "F.Cu") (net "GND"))
 (segment (start 161.976 118.1905) (end 160.964 117.1785) (width 0.2) (layer "F.Cu") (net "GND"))
 (segment (start 121.5 95.053402) (end 121.5 93) (width 0.2) (layer "F.Cu") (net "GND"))
 (segment (start 160.964 117.1785) (end 170.2815 117.1785) (width 0.2) (layer "F.Cu") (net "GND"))
 (segment (start 127.223299 100.776701) (end 121.5 95.053402) (width 0.2) (layer "F.Cu") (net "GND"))
 (segment (start 117 116.6) (end 127.248528 116.6) (width 0.2) (layer "F.Cu") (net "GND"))
 (segment (start 118.5 133.204214) (end 116.669214 135.035) (width 0.2) (layer "F.Cu") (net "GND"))
 (segment (start 116.669214 135.035) (end 115.840786 135.035) (width 0.2) (layer "F.Cu") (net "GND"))
 (segment (start 115.255 118.345) (end 117 116.6) (width 0.2) (layer "F.Cu") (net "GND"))
 (segment (start 127.6 101.153402) (end 127.223299 100.776701) (width 0.2) (layer "F.Cu") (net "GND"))
 (segment (start 115.255 134.449214) (end 115.255 118.345) (width 0.2) (layer "F.Cu") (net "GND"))
 (segment (start 127.6 116.248528) (end 127.6 101.153402) (width 0.2) (layer "F.Cu") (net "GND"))
 (segment (start 173.69 141.96) (end 173.69 115.67) (width 0.2) (layer "B.Cu") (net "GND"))
 (segment (start 173.69 115.67) (end 173.515 115.495) (width 0.2) (layer "B.Cu") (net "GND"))
 (segment (start 127.85 90.46) (end 138.922 90.46) (width 0.2) (layer "F.Cu") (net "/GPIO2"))
 (segment (start 151.04 78.342) (end 153.34 78.342) (width 0.2) (layer "F.Cu") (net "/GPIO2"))
 (segment (start 153.34 78.342) (end 153.34 119.0295) (width 0.2) (layer "F.Cu") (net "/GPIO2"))
 (segment (start 138.922 90.46) (end 151.04 78.342) (width 0.2) (layer "F.Cu") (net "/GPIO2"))
 (segment (start 153.34 119.0295) (end 151.639 120.7305) (width 0.2) (layer "F.Cu") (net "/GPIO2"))
 (segment (start 149.964 131.729142) (end 150.825358 132.5905) (width 0.2) (layer "F.Cu") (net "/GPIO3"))
 (segment (start 151.639 123.2705) (end 149.964 124.9455) (width 0.2) (layer "F.Cu") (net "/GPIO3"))
 (segment (start 173.2105 132.5905) (end 180.04 139.42) (width 0.2) (layer "F.Cu") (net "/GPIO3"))
 (segment (start 150.825358 132.5905) (end 173.2105 132.5905) (width 0.2) (layer "F.Cu") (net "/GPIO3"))
 (segment (start 149.964 124.9455) (end 149.964 131.729142) (width 0.2) (layer "F.Cu") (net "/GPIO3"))
 (segment (start 173.115 111.805) (end 165.663846 111.805) (width 0.2) (layer "F.Cu") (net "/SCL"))
 (segment (start 165.663846 111.805) (end 161.440346 116.0285) (width 0.2) (layer "F.Cu") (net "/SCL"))
 (segment (start 173.515 112.205) (end 173.115 111.805) (width 0.2) (layer "F.Cu") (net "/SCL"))
 (segment (start 171.965 118.035) (end 173.515 116.485) (width 0.2) (layer "F.Cu") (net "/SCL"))
 (segment (start 173.515 116.485) (end 173.515 112.205) (width 0.2) (layer "F.Cu") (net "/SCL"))
 (segment (start 160.487654 116.0285) (end 159.814 116.702154) (width 0.2) (layer "F.Cu") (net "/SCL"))
 (segment (start 154.397792 125.8105) (end 151.639 125.8105) (width 0.2) (layer "F.Cu") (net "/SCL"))
 (segment (start 161.440346 116.0285) (end 160.487654 116.0285) (width 0.2) (layer "F.Cu") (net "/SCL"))
 (segment (start 159.814 116.702154) (end 159.814 120.394292) (width 0.2) (layer "F.Cu") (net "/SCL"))
 (segment (start 159.814 120.394292) (end 154.397792 125.8105) (width 0.2) (layer "F.Cu") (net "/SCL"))
 (segment (start 157.27 79.492) (end 157.27 103.34) (width 0.2) (layer "B.Cu") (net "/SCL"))
 (segment (start 157.27 103.34) (end 171.965 118.035) (width 0.2) (layer "B.Cu") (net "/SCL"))
 (segment (start 171.965 120.575) (end 169.479 123.061) (width 0.2) (layer "F.Cu") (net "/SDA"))
 (segment (start 169.479 131.729142) (end 169.017642 132.1905) (width 0.2) (layer "F.Cu") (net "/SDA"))
 (segment (start 169.479 123.061) (end 169.479 131.729142) (width 0.2) (layer "F.Cu") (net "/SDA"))
 (segment (start 155.479 132.1905) (end 151.639 128.3505) (width 0.2) (layer "F.Cu") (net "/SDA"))
 (segment (start 169.017642 132.1905) (end 155.479 132.1905) (width 0.2) (layer "F.Cu") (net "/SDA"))
 (segment (start 173.115 119.425) (end 171.965 120.575) (width 0.2) (layer "B.Cu") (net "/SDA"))
 (segment (start 173.115 92.797) (end 173.115 119.425) (width 0.2) (layer "B.Cu") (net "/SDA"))
 (segment (start 159.81 79.492) (end 173.115 92.797) (width 0.2) (layer "B.Cu") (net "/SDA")))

